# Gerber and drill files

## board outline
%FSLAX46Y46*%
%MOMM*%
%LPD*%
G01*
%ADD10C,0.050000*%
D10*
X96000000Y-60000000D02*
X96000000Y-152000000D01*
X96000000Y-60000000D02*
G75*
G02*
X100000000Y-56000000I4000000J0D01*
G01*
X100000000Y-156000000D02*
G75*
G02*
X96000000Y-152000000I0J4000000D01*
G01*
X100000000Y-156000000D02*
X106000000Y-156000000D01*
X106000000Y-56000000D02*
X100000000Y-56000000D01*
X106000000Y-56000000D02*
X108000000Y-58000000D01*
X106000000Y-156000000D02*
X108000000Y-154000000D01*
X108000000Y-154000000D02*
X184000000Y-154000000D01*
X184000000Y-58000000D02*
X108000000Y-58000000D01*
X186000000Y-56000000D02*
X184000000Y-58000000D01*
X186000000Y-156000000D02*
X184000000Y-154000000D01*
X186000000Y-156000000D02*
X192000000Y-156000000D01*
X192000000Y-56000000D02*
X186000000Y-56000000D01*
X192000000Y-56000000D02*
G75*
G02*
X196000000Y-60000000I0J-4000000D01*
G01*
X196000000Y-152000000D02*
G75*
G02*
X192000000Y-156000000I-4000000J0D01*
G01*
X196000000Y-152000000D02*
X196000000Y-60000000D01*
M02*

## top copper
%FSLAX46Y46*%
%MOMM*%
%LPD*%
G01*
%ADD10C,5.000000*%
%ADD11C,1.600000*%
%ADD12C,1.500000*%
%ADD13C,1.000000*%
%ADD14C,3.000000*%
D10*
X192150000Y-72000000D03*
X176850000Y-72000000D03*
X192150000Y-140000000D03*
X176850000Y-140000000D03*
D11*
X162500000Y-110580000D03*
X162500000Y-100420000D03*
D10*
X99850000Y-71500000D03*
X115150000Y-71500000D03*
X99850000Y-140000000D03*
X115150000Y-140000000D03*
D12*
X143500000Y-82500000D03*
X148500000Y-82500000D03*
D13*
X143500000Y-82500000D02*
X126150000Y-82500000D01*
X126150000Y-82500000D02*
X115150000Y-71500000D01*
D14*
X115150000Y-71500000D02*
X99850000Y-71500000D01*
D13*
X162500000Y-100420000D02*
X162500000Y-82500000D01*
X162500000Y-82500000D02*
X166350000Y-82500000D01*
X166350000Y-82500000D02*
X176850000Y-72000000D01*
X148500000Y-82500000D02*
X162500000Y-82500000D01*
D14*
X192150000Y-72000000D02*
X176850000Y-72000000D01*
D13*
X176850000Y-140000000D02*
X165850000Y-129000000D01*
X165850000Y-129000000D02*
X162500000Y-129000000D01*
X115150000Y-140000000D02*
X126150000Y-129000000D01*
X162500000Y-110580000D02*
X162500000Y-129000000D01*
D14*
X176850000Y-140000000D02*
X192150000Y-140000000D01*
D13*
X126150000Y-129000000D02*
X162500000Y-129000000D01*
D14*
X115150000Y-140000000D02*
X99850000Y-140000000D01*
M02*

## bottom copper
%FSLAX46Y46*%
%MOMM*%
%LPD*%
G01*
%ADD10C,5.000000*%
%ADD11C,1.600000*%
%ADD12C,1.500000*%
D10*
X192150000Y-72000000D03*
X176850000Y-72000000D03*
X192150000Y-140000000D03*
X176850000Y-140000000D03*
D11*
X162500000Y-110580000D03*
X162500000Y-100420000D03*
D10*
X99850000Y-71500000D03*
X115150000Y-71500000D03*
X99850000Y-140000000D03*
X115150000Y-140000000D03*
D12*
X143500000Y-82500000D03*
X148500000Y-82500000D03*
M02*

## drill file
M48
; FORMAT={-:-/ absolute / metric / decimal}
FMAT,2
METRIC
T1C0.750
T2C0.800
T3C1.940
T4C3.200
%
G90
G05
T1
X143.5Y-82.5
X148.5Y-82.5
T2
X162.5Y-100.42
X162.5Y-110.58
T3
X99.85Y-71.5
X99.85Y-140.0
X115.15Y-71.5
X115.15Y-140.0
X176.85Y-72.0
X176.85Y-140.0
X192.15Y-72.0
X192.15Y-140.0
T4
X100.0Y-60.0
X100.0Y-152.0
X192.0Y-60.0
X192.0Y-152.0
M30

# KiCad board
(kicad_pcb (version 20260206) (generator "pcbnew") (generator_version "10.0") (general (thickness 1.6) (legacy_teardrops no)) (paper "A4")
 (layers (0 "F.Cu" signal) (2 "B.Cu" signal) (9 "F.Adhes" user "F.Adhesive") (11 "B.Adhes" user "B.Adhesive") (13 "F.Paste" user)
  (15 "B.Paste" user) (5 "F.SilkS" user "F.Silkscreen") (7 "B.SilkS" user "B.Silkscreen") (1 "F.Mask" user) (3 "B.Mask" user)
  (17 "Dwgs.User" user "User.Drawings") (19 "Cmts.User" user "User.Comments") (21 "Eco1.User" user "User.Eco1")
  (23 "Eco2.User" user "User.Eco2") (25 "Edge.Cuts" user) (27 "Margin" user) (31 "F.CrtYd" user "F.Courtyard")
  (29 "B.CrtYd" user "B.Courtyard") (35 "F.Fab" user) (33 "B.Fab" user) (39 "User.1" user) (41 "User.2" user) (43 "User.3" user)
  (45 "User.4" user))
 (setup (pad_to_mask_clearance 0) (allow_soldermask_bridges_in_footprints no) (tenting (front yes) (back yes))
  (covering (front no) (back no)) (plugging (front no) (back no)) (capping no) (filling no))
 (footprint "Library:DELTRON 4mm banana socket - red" (layer "F.Cu") (at 184.5 72 180)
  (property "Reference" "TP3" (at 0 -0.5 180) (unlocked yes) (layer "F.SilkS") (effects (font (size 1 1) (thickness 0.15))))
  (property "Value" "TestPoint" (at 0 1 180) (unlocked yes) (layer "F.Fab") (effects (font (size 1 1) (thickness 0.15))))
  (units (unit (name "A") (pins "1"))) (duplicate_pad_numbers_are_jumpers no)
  (pad "1" thru_hole circle (at -7.65 0 180) (size 5 5) (drill 1.94) (layers "*.Cu" "*.Mask") (remove_unused_layers no)
   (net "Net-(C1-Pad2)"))
  (pad "1" thru_hole circle (at 7.65 0 180) (size 5 5) (drill 1.94) (layers "*.Cu" "*.Mask") (remove_unused_layers no) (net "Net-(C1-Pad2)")))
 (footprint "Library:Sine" (layer "F.Cu") (at 115 111)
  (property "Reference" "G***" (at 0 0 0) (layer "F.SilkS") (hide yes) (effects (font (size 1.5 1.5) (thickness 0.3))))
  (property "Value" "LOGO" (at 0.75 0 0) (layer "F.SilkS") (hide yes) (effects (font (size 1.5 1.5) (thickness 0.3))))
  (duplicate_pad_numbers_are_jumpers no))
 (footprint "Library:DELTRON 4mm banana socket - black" (layer "F.Cu") (at 184.5 140 180)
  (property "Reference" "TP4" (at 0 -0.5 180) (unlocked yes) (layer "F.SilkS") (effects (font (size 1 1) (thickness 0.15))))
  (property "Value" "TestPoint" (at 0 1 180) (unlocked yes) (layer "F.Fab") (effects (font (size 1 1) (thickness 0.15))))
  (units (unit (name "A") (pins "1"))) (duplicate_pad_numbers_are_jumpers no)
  (pad "1" thru_hole circle (at -7.65 0 180) (size 5 5) (drill 1.94) (layers "*.Cu" "*.Mask") (remove_unused_layers no)
   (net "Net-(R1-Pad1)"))
  (pad "1" thru_hole circle (at 7.65 0 180) (size 5 5) (drill 1.94) (layers "*.Cu" "*.Mask") (remove_unused_layers no) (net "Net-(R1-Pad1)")))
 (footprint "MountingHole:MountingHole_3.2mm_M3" (layer "F.Cu") (at 192 152)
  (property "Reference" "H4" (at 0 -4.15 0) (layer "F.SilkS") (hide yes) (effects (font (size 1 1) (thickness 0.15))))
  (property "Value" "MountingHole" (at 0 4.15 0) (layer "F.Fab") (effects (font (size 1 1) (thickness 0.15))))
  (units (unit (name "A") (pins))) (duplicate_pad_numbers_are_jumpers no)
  (pad "" np_thru_hole circle (at 0 0) (size 3.2 3.2) (drill 3.2) (layers "*.Cu" "*.Mask")))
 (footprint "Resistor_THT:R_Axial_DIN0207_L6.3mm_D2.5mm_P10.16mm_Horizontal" (layer "F.Cu") (at 162.5 110.58 90)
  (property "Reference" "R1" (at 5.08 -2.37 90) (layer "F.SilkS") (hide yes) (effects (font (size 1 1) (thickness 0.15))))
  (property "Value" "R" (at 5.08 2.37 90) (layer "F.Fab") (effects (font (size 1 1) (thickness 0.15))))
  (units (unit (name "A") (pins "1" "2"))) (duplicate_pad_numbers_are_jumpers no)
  (pad "1" thru_hole circle (at 0 0 90) (size 1.6 1.6) (drill 0.8) (layers "*.Cu" "*.Mask") (remove_unused_layers no) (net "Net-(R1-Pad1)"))
  (pad "2" thru_hole circle (at 10.16 0 90) (size 1.6 1.6) (drill 0.8) (layers "*.Cu" "*.Mask") (remove_unused_layers no)
   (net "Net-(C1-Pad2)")))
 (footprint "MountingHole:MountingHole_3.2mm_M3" (layer "F.Cu") (at 100 152)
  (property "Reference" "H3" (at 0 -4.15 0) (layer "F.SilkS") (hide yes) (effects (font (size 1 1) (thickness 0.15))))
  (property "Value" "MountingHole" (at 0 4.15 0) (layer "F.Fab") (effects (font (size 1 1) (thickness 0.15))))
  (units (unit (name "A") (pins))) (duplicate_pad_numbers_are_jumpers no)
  (pad "" np_thru_hole circle (at 0 0) (size 3.2 3.2) (drill 3.2) (layers "*.Cu" "*.Mask")))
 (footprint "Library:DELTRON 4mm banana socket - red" (layer "F.Cu") (at 107.5 71.5)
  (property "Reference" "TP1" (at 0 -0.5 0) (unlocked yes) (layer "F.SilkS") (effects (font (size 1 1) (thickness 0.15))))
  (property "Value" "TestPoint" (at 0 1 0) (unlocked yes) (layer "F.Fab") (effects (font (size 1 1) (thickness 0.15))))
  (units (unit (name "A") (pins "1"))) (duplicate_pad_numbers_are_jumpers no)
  (pad "1" thru_hole circle (at -7.65 0) (size 5 5) (drill 1.94) (layers "*.Cu" "*.Mask") (remove_unused_layers no) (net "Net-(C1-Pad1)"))
  (pad "1" thru_hole circle (at 7.65 0) (size 5 5) (drill 1.94) (layers "*.Cu" "*.Mask") (remove_unused_layers no) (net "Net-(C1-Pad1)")))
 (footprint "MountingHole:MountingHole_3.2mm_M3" (layer "F.Cu") (at 100 60)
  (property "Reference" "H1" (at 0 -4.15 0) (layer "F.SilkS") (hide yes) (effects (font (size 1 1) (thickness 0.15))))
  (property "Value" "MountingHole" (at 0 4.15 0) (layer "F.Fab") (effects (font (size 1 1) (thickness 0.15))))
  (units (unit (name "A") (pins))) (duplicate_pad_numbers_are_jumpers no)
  (pad "" np_thru_hole circle (at 0 0) (size 3.2 3.2) (drill 3.2) (layers "*.Cu" "*.Mask")))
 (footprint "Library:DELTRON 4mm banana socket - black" (layer "F.Cu") (at 107.5 140)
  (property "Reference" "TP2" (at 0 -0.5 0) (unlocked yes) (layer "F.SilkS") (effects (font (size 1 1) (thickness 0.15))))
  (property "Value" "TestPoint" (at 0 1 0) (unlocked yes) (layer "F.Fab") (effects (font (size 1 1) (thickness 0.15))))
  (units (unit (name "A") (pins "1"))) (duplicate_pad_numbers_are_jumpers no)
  (pad "1" thru_hole circle (at -7.65 0) (size 5 5) (drill 1.94) (layers "*.Cu" "*.Mask") (remove_unused_layers no) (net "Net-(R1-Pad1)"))
  (pad "1" thru_hole circle (at 7.65 0) (size 5 5) (drill 1.94) (layers "*.Cu" "*.Mask") (remove_unused_layers no) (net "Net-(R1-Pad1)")))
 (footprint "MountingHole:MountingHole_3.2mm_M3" (layer "F.Cu") (at 192 60)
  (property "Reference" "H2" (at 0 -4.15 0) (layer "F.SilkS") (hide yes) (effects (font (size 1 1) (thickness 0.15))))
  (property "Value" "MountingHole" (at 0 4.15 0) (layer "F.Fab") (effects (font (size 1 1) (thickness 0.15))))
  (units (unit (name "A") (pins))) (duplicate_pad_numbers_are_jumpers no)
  (pad "" np_thru_hole circle (at 0 0) (size 3.2 3.2) (drill 3.2) (layers "*.Cu" "*.Mask")))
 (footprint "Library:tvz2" (layer "F.Cu") (at 146 63.959347)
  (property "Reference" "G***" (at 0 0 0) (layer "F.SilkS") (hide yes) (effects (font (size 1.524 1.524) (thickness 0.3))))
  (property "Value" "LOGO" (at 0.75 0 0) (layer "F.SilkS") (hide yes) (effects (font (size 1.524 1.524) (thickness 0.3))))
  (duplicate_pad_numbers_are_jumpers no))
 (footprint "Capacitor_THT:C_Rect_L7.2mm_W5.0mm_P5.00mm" (layer "F.Cu") (at 143.5 82.5)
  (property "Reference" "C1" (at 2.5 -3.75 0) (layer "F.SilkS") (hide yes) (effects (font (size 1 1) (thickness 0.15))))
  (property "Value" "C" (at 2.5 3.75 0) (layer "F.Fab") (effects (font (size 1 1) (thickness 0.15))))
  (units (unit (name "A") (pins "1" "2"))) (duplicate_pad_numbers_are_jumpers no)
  (pad "1" thru_hole circle (at 0 0) (size 1.5 1.5) (drill 0.75) (layers "*.Cu" "*.Mask") (remove_unused_layers no) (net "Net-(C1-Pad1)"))
  (pad "2" thru_hole circle (at 5 0) (size 1.5 1.5) (drill 0.75) (layers "*.Cu" "*.Mask") (remove_unused_layers no) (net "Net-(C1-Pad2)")))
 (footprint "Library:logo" (layer "B.Cu") (at 180.5 149 180)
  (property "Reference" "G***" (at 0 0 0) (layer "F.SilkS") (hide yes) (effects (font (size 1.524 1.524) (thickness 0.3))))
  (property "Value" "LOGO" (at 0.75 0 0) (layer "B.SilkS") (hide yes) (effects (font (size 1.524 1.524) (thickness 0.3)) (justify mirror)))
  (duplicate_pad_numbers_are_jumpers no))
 (gr_line (start 96 60) (end 96 152) (stroke (width 0.05) (type default)) (layer "Edge.Cuts"))
 (gr_arc (start 96 60) (mid 97.171573 57.171573) (end 100 56) (stroke (width 0.05) (type default)) (layer "Edge.Cuts"))
 (gr_arc (start 100 156) (mid 97.171573 154.828427) (end 96 152) (stroke (width 0.05) (type default)) (layer "Edge.Cuts"))
 (gr_line (start 100 156) (end 106 156) (stroke (width 0.05) (type default)) (layer "Edge.Cuts"))
 (gr_line (start 106 56) (end 100 56) (stroke (width 0.05) (type default)) (layer "Edge.Cuts"))
 (gr_line (start 106 56) (end 108 58) (stroke (width 0.05) (type default)) (layer "Edge.Cuts"))
 (gr_line (start 106 156) (end 108 154) (stroke (width 0.05) (type default)) (layer "Edge.Cuts"))
 (gr_line (start 108 154) (end 184 154) (stroke (width 0.05) (type default)) (layer "Edge.Cuts"))
 (gr_line (start 184 58) (end 108 58) (stroke (width 0.05) (type default)) (layer "Edge.Cuts"))
 (gr_line (start 186 56) (end 184 58) (stroke (width 0.05) (type default)) (layer "Edge.Cuts"))
 (gr_line (start 186 156) (end 184 154) (stroke (width 0.05) (type default)) (layer "Edge.Cuts"))
 (gr_line (start 186 156) (end 192 156) (stroke (width 0.05) (type default)) (layer "Edge.Cuts"))
 (gr_line (start 192 56) (end 186 56) (stroke (width 0.05) (type default)) (layer "Edge.Cuts"))
 (gr_arc (start 192 56) (mid 194.828427 57.171573) (end 196 60) (stroke (width 0.05) (type default)) (layer "Edge.Cuts"))
 (gr_arc (start 196 152) (mid 194.828427 154.828427) (end 192 156) (stroke (width 0.05) (type default)) (layer "Edge.Cuts"))
 (gr_line (start 196 152) (end 196 60) (stroke (width 0.05) (type default)) (layer "Edge.Cuts"))
 (segment (start 143.5 82.5) (end 126.15 82.5) (width 1) (layer "F.Cu") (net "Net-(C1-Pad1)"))
 (segment (start 126.15 82.5) (end 115.15 71.5) (width 1) (layer "F.Cu") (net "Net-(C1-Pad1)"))
 (segment (start 115.15 71.5) (end 99.85 71.5) (width 3) (layer "F.Cu") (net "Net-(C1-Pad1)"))
 (segment (start 162.5 100.42) (end 162.5 82.5) (width 1) (layer "F.Cu") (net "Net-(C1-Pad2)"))
 (segment (start 162.5 82.5) (end 166.35 82.5) (width 1) (layer "F.Cu") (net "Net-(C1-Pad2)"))
 (segment (start 166.35 82.5) (end 176.85 72) (width 1) (layer "F.Cu") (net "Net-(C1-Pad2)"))
 (segment (start 148.5 82.5) (end 162.5 82.5) (width 1) (layer "F.Cu") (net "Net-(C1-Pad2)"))
 (segment (start 192.15 72) (end 176.85 72) (width 3) (layer "F.Cu") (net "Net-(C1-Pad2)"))
 (segment (start 176.85 140) (end 165.85 129) (width 1) (layer "F.Cu") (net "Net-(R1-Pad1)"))
 (segment (start 165.85 129) (end 162.5 129) (width 1) (layer "F.Cu") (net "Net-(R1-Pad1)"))
 (segment (start 115.15 140) (end 126.15 129) (width 1) (layer "F.Cu") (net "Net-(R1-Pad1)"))
 (segment (start 162.5 110.58) (end 162.5 129) (width 1) (layer "F.Cu") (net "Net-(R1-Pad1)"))
 (segment (start 176.85 140) (end 192.15 140) (width 3) (layer "F.Cu") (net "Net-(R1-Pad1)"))
 (segment (start 126.15 129) (end 162.5 129) (width 1) (layer "F.Cu") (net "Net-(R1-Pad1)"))
 (segment (start 115.15 140) (end 99.85 140) (width 3) (layer "F.Cu") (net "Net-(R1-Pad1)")))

